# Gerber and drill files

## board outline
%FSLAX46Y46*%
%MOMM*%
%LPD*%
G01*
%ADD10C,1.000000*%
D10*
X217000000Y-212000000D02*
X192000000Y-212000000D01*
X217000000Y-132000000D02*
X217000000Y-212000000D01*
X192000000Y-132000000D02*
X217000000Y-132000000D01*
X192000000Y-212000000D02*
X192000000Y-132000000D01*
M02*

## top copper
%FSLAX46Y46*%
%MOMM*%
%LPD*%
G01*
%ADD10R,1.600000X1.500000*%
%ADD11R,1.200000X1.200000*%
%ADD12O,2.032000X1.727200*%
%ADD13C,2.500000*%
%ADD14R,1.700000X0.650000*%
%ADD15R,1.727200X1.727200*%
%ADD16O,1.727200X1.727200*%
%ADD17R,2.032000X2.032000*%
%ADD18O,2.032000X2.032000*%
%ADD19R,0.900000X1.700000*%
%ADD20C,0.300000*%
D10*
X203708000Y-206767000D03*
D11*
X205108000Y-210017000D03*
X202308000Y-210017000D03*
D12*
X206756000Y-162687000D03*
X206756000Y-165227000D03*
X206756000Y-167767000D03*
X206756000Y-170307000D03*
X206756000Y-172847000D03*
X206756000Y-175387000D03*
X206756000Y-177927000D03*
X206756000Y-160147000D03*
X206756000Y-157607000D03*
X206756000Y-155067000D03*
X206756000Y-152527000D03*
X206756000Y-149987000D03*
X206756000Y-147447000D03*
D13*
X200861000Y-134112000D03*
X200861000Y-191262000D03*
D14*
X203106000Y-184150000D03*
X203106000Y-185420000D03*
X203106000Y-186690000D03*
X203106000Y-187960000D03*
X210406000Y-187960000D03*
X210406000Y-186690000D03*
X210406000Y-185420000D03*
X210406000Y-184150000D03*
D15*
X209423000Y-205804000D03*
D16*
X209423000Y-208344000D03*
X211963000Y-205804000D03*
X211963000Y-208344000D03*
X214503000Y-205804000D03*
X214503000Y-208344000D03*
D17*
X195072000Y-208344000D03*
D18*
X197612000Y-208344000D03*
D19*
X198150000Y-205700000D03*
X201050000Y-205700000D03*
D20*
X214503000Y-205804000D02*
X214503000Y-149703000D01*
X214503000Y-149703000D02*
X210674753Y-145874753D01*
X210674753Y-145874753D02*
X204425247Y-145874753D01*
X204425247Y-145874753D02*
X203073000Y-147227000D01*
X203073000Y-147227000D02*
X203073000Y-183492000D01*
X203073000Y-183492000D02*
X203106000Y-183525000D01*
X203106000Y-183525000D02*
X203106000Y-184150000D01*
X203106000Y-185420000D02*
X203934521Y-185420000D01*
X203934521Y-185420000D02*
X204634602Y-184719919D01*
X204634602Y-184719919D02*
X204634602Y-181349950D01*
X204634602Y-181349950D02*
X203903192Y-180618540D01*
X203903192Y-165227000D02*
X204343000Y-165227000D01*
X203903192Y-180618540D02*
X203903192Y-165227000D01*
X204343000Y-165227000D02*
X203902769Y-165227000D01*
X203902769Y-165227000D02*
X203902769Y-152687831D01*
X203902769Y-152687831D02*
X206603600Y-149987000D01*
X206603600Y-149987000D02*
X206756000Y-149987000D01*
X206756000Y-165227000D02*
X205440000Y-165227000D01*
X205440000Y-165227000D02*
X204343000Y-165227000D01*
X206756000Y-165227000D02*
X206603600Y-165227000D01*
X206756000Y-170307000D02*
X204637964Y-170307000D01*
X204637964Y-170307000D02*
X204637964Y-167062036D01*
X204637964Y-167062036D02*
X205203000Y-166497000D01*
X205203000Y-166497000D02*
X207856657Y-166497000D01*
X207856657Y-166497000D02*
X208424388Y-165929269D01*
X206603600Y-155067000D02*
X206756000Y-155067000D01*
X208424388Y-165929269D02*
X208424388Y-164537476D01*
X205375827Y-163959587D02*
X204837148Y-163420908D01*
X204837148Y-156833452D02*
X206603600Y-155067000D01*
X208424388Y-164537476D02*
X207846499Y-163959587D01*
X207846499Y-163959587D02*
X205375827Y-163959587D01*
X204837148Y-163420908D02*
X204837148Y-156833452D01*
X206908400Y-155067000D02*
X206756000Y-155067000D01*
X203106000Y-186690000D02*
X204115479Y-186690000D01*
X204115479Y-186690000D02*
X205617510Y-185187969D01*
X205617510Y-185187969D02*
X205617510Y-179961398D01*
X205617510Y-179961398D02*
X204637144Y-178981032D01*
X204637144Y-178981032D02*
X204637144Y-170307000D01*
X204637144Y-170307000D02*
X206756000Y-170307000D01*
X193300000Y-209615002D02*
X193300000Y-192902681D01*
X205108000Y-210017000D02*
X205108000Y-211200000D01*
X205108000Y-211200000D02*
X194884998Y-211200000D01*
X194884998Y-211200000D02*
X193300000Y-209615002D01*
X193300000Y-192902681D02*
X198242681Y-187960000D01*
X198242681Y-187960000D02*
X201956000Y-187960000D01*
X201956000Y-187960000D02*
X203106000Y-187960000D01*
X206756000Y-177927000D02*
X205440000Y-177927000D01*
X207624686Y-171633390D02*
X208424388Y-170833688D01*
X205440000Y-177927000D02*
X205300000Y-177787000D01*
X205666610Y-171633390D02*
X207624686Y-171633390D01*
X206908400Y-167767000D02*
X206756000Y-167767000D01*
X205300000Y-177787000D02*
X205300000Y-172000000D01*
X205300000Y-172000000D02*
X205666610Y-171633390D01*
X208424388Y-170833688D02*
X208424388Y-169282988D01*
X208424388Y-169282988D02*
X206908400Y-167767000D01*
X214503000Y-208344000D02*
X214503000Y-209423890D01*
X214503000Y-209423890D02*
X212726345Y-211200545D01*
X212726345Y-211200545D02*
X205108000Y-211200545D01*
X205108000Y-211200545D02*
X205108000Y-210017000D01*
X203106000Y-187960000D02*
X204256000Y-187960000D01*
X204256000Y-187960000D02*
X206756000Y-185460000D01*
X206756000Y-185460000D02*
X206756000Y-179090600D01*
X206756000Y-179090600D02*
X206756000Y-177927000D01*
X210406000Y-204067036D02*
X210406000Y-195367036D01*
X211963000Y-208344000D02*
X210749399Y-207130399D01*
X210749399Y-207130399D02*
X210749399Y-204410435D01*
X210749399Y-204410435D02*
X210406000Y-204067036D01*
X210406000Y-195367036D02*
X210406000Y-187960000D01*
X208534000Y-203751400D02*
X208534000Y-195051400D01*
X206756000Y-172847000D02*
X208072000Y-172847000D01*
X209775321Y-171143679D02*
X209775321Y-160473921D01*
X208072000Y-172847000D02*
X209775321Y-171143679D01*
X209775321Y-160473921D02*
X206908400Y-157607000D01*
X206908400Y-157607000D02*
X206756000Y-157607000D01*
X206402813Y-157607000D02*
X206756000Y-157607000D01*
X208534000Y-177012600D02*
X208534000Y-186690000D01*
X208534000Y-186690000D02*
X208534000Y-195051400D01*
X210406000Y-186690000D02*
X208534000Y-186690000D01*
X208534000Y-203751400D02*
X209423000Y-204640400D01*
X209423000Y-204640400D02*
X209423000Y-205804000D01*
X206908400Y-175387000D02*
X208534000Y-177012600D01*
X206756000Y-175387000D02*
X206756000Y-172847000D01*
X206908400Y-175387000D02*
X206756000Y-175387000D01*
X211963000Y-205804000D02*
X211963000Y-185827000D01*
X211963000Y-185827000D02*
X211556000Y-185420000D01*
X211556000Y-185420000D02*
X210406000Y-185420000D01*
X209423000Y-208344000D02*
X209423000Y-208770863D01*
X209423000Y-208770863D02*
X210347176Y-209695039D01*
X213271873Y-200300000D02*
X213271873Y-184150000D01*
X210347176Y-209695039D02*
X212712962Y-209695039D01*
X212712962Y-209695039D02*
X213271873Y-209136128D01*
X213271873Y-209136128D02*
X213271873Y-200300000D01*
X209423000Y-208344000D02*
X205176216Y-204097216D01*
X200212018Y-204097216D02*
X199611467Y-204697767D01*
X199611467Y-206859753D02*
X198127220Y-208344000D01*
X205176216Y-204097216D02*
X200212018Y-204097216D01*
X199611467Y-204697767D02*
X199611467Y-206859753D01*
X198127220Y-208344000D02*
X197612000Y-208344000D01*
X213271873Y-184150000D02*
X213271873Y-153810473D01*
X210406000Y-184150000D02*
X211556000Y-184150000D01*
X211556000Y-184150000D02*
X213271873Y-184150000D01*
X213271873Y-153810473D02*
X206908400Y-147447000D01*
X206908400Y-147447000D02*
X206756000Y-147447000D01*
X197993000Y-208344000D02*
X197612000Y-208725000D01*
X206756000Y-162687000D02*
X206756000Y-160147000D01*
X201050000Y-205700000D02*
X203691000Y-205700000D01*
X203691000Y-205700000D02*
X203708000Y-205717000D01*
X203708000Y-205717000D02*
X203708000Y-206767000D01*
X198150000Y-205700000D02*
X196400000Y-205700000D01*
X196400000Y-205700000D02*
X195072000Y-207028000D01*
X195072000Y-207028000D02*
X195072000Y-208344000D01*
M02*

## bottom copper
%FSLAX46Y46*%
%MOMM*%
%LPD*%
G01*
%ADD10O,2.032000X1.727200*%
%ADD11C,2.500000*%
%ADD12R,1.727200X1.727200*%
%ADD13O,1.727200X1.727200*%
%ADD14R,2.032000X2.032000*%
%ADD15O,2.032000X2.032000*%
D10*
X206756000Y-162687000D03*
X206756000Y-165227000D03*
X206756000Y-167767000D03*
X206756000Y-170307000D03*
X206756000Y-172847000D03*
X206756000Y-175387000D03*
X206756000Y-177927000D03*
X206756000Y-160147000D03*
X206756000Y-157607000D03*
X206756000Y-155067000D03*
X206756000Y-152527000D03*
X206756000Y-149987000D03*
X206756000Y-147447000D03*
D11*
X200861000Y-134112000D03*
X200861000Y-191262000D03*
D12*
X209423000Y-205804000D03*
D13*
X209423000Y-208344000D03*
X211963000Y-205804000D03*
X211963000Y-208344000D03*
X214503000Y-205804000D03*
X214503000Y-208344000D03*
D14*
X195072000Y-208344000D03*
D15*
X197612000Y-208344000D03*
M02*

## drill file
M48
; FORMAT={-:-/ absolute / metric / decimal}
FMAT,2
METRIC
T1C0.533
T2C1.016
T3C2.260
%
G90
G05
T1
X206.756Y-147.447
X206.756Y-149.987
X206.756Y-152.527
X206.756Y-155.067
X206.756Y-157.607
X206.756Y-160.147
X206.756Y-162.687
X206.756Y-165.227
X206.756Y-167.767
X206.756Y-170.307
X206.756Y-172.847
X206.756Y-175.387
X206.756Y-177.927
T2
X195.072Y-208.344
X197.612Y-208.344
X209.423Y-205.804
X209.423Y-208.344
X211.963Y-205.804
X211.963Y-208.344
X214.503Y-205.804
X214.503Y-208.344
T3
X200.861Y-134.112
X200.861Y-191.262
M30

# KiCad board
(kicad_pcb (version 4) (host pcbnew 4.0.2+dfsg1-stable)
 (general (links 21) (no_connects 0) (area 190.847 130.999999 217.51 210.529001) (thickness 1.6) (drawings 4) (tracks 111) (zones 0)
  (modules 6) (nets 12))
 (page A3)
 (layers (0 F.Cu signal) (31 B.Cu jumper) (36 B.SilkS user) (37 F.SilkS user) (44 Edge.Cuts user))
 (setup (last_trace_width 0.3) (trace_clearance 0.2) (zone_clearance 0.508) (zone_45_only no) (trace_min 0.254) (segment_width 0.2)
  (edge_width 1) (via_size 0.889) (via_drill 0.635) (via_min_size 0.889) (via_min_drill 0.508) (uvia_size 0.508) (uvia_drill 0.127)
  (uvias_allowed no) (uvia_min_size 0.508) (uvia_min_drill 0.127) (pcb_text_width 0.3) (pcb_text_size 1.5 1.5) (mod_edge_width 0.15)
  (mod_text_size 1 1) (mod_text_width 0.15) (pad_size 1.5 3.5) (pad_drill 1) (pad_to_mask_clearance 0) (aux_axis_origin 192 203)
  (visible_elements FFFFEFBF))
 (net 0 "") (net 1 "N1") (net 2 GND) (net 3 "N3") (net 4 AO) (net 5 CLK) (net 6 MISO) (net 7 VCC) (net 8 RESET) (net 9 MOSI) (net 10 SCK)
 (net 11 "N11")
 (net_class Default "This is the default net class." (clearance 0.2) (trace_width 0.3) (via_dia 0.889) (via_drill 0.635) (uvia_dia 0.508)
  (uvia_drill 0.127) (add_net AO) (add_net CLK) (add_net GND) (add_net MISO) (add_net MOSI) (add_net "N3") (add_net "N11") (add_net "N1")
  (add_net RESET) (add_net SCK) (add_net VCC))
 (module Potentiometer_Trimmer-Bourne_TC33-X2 (layer F.Cu) (at 203.708 208.217)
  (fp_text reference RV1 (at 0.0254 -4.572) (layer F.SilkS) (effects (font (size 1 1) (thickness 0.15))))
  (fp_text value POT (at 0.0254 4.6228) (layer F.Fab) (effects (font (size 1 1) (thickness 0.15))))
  (pad 2 smd rect (at 0 -1.45) (size 1.6 1.5) (layers F.Cu) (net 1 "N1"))
  (pad 3 smd rect (at 1.4 1.8) (size 1.2 1.2) (layers F.Cu) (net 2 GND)) (pad 1 smd rect (at -1.4 1.8) (size 1.2 1.2) (layers F.Cu)))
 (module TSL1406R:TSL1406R (layer B.Cu) (at 200.861 162.687)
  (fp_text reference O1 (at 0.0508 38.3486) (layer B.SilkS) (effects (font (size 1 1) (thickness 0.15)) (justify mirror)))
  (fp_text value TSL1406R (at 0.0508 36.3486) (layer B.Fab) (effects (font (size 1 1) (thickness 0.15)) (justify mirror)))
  (pad 7 thru_hole oval (at 5.895 0) (size 2.032 1.7272) (drill 0.533) (layers *.Cu *.Mask B.SilkS) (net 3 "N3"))
  (pad 6 thru_hole oval (at 5.895 2.54) (size 2.032 1.7272) (drill 0.533) (layers *.Cu *.Mask B.SilkS) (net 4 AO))
  (pad 5 thru_hole oval (at 5.895 5.08) (size 2.032 1.7272) (drill 0.533) (layers *.Cu *.Mask B.SilkS) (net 2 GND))
  (pad 4 thru_hole oval (at 5.895 7.62) (size 2.032 1.7272) (drill 0.533) (layers *.Cu *.Mask B.SilkS) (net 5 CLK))
  (pad 3 thru_hole oval (at 5.895 10.16) (size 2.032 1.7272) (drill 0.533) (layers *.Cu *.Mask B.SilkS) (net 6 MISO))
  (pad 2 thru_hole oval (at 5.895 12.7) (size 2.032 1.7272) (drill 0.533) (layers *.Cu *.Mask B.SilkS) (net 6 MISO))
  (pad 1 thru_hole oval (at 5.895 15.24) (size 2.032 1.7272) (drill 0.533) (layers *.Cu *.Mask B.SilkS) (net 2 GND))
  (pad 8 thru_hole oval (at 5.895 -2.54) (size 2.032 1.7272) (drill 0.533) (layers *.Cu *.Mask B.SilkS) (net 3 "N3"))
  (pad 9 thru_hole oval (at 5.895 -5.08) (size 2.032 1.7272) (drill 0.533) (layers *.Cu *.Mask B.SilkS) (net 6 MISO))
  (pad 10 thru_hole oval (at 5.895 -7.62) (size 2.032 1.7272) (drill 0.533) (layers *.Cu *.Mask B.SilkS) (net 5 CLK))
  (pad 11 thru_hole oval (at 5.895 -10.16) (size 2.032 1.7272) (drill 0.533) (layers *.Cu *.Mask B.SilkS))
  (pad 12 thru_hole oval (at 5.895 -12.7) (size 2.032 1.7272) (drill 0.533) (layers *.Cu *.Mask B.SilkS) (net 4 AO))
  (pad 13 thru_hole oval (at 5.895 -15.24) (size 2.032 1.7272) (drill 0.533) (layers *.Cu *.Mask B.SilkS) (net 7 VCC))
  (pad 0 thru_hole circle (at 0 -28.575) (size 2.5 2.5) (drill 2.26) (layers *.Cu *.Mask B.SilkS))
  (pad 0 thru_hole circle (at 0 28.575) (size 2.5 2.5) (drill 2.26) (layers *.Cu *.Mask B.SilkS)))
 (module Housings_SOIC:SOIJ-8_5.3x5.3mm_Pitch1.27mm (layer F.Cu) (at 206.756 186.055)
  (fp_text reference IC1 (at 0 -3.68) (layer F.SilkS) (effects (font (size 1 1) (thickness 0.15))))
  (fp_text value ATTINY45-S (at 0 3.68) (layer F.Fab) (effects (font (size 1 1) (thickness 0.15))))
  (pad 1 smd rect (at -3.65 -1.905) (size 1.7 0.65) (layers F.Cu) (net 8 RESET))
  (pad 2 smd rect (at -3.65 -0.635) (size 1.7 0.65) (layers F.Cu) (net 4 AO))
  (pad 3 smd rect (at -3.65 0.635) (size 1.7 0.65) (layers F.Cu) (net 5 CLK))
  (pad 4 smd rect (at -3.65 1.905) (size 1.7 0.65) (layers F.Cu) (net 2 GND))
  (pad 5 smd rect (at 3.65 1.905) (size 1.7 0.65) (layers F.Cu) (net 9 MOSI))
  (pad 6 smd rect (at 3.65 0.635) (size 1.7 0.65) (layers F.Cu) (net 6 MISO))
  (pad 7 smd rect (at 3.65 -0.635) (size 1.7 0.65) (layers F.Cu) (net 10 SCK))
  (pad 8 smd rect (at 3.65 -1.905) (size 1.7 0.65) (layers F.Cu) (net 7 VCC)))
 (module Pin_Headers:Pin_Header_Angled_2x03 (layer B.Cu) (at 209.423 205.804 270)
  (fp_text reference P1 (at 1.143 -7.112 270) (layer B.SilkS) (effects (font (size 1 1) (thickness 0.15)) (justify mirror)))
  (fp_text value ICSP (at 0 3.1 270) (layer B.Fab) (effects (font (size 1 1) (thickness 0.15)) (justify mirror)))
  (pad 1 thru_hole rect (at 0 0 270) (size 1.7272 1.7272) (drill 1.016) (layers *.Cu *.Mask B.SilkS) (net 6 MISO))
  (pad 2 thru_hole oval (at 2.54 0 270) (size 1.7272 1.7272) (drill 1.016) (layers *.Cu *.Mask B.SilkS) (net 7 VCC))
  (pad 3 thru_hole oval (at 0 -2.54 270) (size 1.7272 1.7272) (drill 1.016) (layers *.Cu *.Mask B.SilkS) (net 10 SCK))
  (pad 4 thru_hole oval (at 2.54 -2.54 270) (size 1.7272 1.7272) (drill 1.016) (layers *.Cu *.Mask B.SilkS) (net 9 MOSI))
  (pad 5 thru_hole oval (at 0 -5.08 270) (size 1.7272 1.7272) (drill 1.016) (layers *.Cu *.Mask B.SilkS) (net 8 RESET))
  (pad 6 thru_hole oval (at 2.54 -5.08 270) (size 1.7272 1.7272) (drill 1.016) (layers *.Cu *.Mask B.SilkS) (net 2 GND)))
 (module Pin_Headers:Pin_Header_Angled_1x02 (layer B.Cu) (at 195.072 208.344 270)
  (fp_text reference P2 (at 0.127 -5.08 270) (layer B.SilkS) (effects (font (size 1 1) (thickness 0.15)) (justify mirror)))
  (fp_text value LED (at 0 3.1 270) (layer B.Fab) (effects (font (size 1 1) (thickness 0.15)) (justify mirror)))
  (pad 1 thru_hole rect (at 0 0 270) (size 2.032 2.032) (drill 1.016) (layers *.Cu *.Mask B.SilkS) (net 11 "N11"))
  (pad 2 thru_hole oval (at 0 -2.54 270) (size 2.032 2.032) (drill 1.016) (layers *.Cu *.Mask B.SilkS) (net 7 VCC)))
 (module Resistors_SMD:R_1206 (layer F.Cu) (at 199.6 205.7)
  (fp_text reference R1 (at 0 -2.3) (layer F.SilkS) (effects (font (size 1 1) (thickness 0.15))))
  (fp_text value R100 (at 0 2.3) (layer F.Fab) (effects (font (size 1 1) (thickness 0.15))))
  (pad 1 smd rect (at -1.45 0) (size 0.9 1.7) (layers F.Cu) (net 11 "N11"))
  (pad 2 smd rect (at 1.45 0) (size 0.9 1.7) (layers F.Cu) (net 1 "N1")))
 (gr_line (start 217 212) (end 192 212) (layer Edge.Cuts) (width 1))
 (gr_line (start 217 132) (end 217 212) (layer Edge.Cuts) (width 1))
 (gr_line (start 192 132) (end 217 132) (layer Edge.Cuts) (width 1))
 (gr_line (start 192 212) (end 192 132) (layer Edge.Cuts) (width 1))
 (segment (start 214.503 205.804) (end 214.503 149.703) (width 0.3) (layer F.Cu) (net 8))
 (segment (start 214.503 149.703) (end 210.674753 145.874753) (width 0.3) (layer F.Cu) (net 8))
 (segment (start 210.674753 145.874753) (end 204.425247 145.874753) (width 0.3) (layer F.Cu) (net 8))
 (segment (start 204.425247 145.874753) (end 203.073 147.227) (width 0.3) (layer F.Cu) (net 8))
 (segment (start 203.073 147.227) (end 203.073 183.492) (width 0.3) (layer F.Cu) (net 8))
 (segment (start 203.073 183.492) (end 203.106 183.525) (width 0.3) (layer F.Cu) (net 8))
 (segment (start 203.106 183.525) (end 203.106 184.15) (width 0.3) (layer F.Cu) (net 8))
 (segment (start 203.106 185.42) (end 203.934521 185.42) (width 0.3) (layer F.Cu) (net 4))
 (segment (start 203.934521 185.42) (end 204.634602 184.719919) (width 0.3) (layer F.Cu) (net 4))
 (segment (start 204.634602 184.719919) (end 204.634602 181.34995) (width 0.3) (layer F.Cu) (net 4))
 (segment (start 204.634602 181.34995) (end 203.903192 180.61854) (width 0.3) (layer F.Cu) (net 4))
 (segment (start 203.903192 165.227) (end 204.343 165.227) (width 0.3) (layer F.Cu) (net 4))
 (segment (start 203.903192 180.61854) (end 203.903192 165.227) (width 0.3) (layer F.Cu) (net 4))
 (segment (start 204.343 165.227) (end 203.902769 165.227) (width 0.3) (layer F.Cu) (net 4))
 (segment (start 203.902769 165.227) (end 203.902769 152.687831) (width 0.3) (layer F.Cu) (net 4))
 (segment (start 203.902769 152.687831) (end 206.6036 149.987) (width 0.3) (layer F.Cu) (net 4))
 (segment (start 206.6036 149.987) (end 206.756 149.987) (width 0.3) (layer F.Cu) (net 4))
 (segment (start 206.756 165.227) (end 205.44 165.227) (width 0.3) (layer F.Cu) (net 4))
 (segment (start 205.44 165.227) (end 204.343 165.227) (width 0.3) (layer F.Cu) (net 4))
 (segment (start 206.756 165.227) (end 206.6036 165.227) (width 0.3) (layer F.Cu) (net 4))
 (segment (start 206.756 170.307) (end 204.637964 170.307) (width 0.3) (layer F.Cu) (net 5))
 (segment (start 204.637964 170.307) (end 204.637964 167.062036) (width 0.3) (layer F.Cu) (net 5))
 (segment (start 204.637964 167.062036) (end 205.203 166.497) (width 0.3) (layer F.Cu) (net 5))
 (segment (start 205.203 166.497) (end 207.856657 166.497) (width 0.3) (layer F.Cu) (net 5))
 (segment (start 207.856657 166.497) (end 208.424388 165.929269) (width 0.3) (layer F.Cu) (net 5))
 (segment (start 206.6036 155.067) (end 206.756 155.067) (width 0.3) (layer F.Cu) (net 5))
 (segment (start 208.424388 165.929269) (end 208.424388 164.537476) (width 0.3) (layer F.Cu) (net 5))
 (segment (start 205.375827 163.959587) (end 204.837148 163.420908) (width 0.3) (layer F.Cu) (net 5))
 (segment (start 204.837148 156.833452) (end 206.6036 155.067) (width 0.3) (layer F.Cu) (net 5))
 (segment (start 208.424388 164.537476) (end 207.846499 163.959587) (width 0.3) (layer F.Cu) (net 5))
 (segment (start 207.846499 163.959587) (end 205.375827 163.959587) (width 0.3) (layer F.Cu) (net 5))
 (segment (start 204.837148 163.420908) (end 204.837148 156.833452) (width 0.3) (layer F.Cu) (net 5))
 (segment (start 206.9084 155.067) (end 206.756 155.067) (width 0.3) (layer F.Cu) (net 5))
 (segment (start 203.106 186.69) (end 204.115479 186.69) (width 0.3) (layer F.Cu) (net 5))
 (segment (start 204.115479 186.69) (end 205.61751 185.187969) (width 0.3) (layer F.Cu) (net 5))
 (segment (start 205.61751 185.187969) (end 205.61751 179.961398) (width 0.3) (layer F.Cu) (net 5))
 (segment (start 205.61751 179.961398) (end 204.637144 178.981032) (width 0.3) (layer F.Cu) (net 5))
 (segment (start 204.637144 178.981032) (end 204.637144 170.307) (width 0.3) (layer F.Cu) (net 5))
 (segment (start 204.637144 170.307) (end 206.756 170.307) (width 0.3) (layer F.Cu) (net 5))
 (segment (start 193.3 209.615002) (end 193.3 192.902681) (width 0.3) (layer F.Cu) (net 2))
 (segment (start 205.108 210.017) (end 205.108 211.2) (width 0.3) (layer F.Cu) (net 2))
 (segment (start 205.108 211.2) (end 194.884998 211.2) (width 0.3) (layer F.Cu) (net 2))
 (segment (start 194.884998 211.2) (end 193.3 209.615002) (width 0.3) (layer F.Cu) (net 2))
 (segment (start 193.3 192.902681) (end 198.242681 187.96) (width 0.3) (layer F.Cu) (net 2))
 (segment (start 198.242681 187.96) (end 201.956 187.96) (width 0.3) (layer F.Cu) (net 2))
 (segment (start 201.956 187.96) (end 203.106 187.96) (width 0.3) (layer F.Cu) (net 2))
 (segment (start 206.756 177.927) (end 205.44 177.927) (width 0.3) (layer F.Cu) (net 2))
 (segment (start 207.624686 171.63339) (end 208.424388 170.833688) (width 0.3) (layer F.Cu) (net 2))
 (segment (start 205.44 177.927) (end 205.3 177.787) (width 0.3) (layer F.Cu) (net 2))
 (segment (start 205.66661 171.63339) (end 207.624686 171.63339) (width 0.3) (layer F.Cu) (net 2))
 (segment (start 206.9084 167.767) (end 206.756 167.767) (width 0.3) (layer F.Cu) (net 2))
 (segment (start 205.3 177.787) (end 205.3 172) (width 0.3) (layer F.Cu) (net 2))
 (segment (start 205.3 172) (end 205.66661 171.63339) (width 0.3) (layer F.Cu) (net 2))
 (segment (start 208.424388 170.833688) (end 208.424388 169.282988) (width 0.3) (layer F.Cu) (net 2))
 (segment (start 208.424388 169.282988) (end 206.9084 167.767) (width 0.3) (layer F.Cu) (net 2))
 (segment (start 214.503 208.344) (end 214.503 209.42389) (width 0.3) (layer F.Cu) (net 2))
 (segment (start 214.503 209.42389) (end 212.726345 211.200545) (width 0.3) (layer F.Cu) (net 2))
 (segment (start 212.726345 211.200545) (end 205.108 211.200545) (width 0.3) (layer F.Cu) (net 2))
 (segment (start 205.108 211.200545) (end 205.108 210.017) (width 0.3) (layer F.Cu) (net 2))
 (segment (start 203.106 187.96) (end 204.256 187.96) (width 0.3) (layer F.Cu) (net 2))
 (segment (start 204.256 187.96) (end 206.756 185.46) (width 0.3) (layer F.Cu) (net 2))
 (segment (start 206.756 185.46) (end 206.756 179.0906) (width 0.3) (layer F.Cu) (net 2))
 (segment (start 206.756 179.0906) (end 206.756 177.927) (width 0.3) (layer F.Cu) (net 2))
 (segment (start 210.406 204.067036) (end 210.406 195.367036) (width 0.3) (layer F.Cu) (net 9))
 (segment (start 211.963 208.344) (end 210.749399 207.130399) (width 0.3) (layer F.Cu) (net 9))
 (segment (start 210.749399 207.130399) (end 210.749399 204.410435) (width 0.3) (layer F.Cu) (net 9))
 (segment (start 210.749399 204.410435) (end 210.406 204.067036) (width 0.3) (layer F.Cu) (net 9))
 (segment (start 210.406 195.367036) (end 210.406 187.96) (width 0.3) (layer F.Cu) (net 9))
 (segment (start 208.534 203.7514) (end 208.534 195.0514) (width 0.3) (layer F.Cu) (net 6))
 (segment (start 206.756 172.847) (end 208.072 172.847) (width 0.3) (layer F.Cu) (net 6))
 (segment (start 209.775321 171.143679) (end 209.775321 160.473921) (width 0.3) (layer F.Cu) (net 6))
 (segment (start 208.072 172.847) (end 209.775321 171.143679) (width 0.3) (layer F.Cu) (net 6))
 (segment (start 209.775321 160.473921) (end 206.9084 157.607) (width 0.3) (layer F.Cu) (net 6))
 (segment (start 206.9084 157.607) (end 206.756 157.607) (width 0.3) (layer F.Cu) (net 6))
 (segment (start 206.402813 157.607) (end 206.756 157.607) (width 0.3) (layer F.Cu) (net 6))
 (segment (start 208.534 177.0126) (end 208.534 186.69) (width 0.3) (layer F.Cu) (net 6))
 (segment (start 208.534 186.69) (end 208.534 195.0514) (width 0.3) (layer F.Cu) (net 6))
 (segment (start 210.406 186.69) (end 208.534 186.69) (width 0.3) (layer F.Cu) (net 6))
 (segment (start 208.534 203.7514) (end 209.423 204.6404) (width 0.3) (layer F.Cu) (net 6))
 (segment (start 209.423 204.6404) (end 209.423 205.804) (width 0.3) (layer F.Cu) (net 6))
 (segment (start 206.9084 175.387) (end 208.534 177.0126) (width 0.3) (layer F.Cu) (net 6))
 (segment (start 206.756 175.387) (end 206.756 172.847) (width 0.3) (layer F.Cu) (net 6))
 (segment (start 206.9084 175.387) (end 206.756 175.387) (width 0.3) (layer F.Cu) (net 6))
 (segment (start 211.963 205.804) (end 211.963 185.827) (width 0.3) (layer F.Cu) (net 10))
 (segment (start 211.963 185.827) (end 211.556 185.42) (width 0.3) (layer F.Cu) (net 10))
 (segment (start 211.556 185.42) (end 210.406 185.42) (width 0.3) (layer F.Cu) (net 10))
 (segment (start 209.423 208.344) (end 209.423 208.770863) (width 0.3) (layer F.Cu) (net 7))
 (segment (start 209.423 208.770863) (end 210.347176 209.695039) (width 0.3) (layer F.Cu) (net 7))
 (segment (start 213.271873 200.3) (end 213.271873 184.15) (width 0.3) (layer F.Cu) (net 7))
 (segment (start 210.347176 209.695039) (end 212.712962 209.695039) (width 0.3) (layer F.Cu) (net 7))
 (segment (start 212.712962 209.695039) (end 213.271873 209.136128) (width 0.3) (layer F.Cu) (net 7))
 (segment (start 213.271873 209.136128) (end 213.271873 200.3) (width 0.3) (layer F.Cu) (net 7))
 (segment (start 209.423 208.344) (end 205.176216 204.097216) (width 0.3) (layer F.Cu) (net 7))
 (segment (start 200.212018 204.097216) (end 199.611467 204.697767) (width 0.3) (layer F.Cu) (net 7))
 (segment (start 199.611467 206.859753) (end 198.12722 208.344) (width 0.3) (layer F.Cu) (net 7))
 (segment (start 205.176216 204.097216) (end 200.212018 204.097216) (width 0.3) (layer F.Cu) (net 7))
 (segment (start 199.611467 204.697767) (end 199.611467 206.859753) (width 0.3) (layer F.Cu) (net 7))
 (segment (start 198.12722 208.344) (end 197.612 208.344) (width 0.3) (layer F.Cu) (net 7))
 (segment (start 213.271873 184.15) (end 213.271873 153.810473) (width 0.3) (layer F.Cu) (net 7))
 (segment (start 210.406 184.15) (end 211.556 184.15) (width 0.3) (layer F.Cu) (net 7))
 (segment (start 211.556 184.15) (end 213.271873 184.15) (width 0.3) (layer F.Cu) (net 7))
 (segment (start 213.271873 153.810473) (end 206.9084 147.447) (width 0.3) (layer F.Cu) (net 7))
 (segment (start 206.9084 147.447) (end 206.756 147.447) (width 0.3) (layer F.Cu) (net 7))
 (segment (start 197.993 208.344) (end 197.612 208.725) (width 0.3) (layer F.Cu) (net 7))
 (segment (start 206.756 162.687) (end 206.756 160.147) (width 0.3) (layer F.Cu) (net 3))
 (segment (start 201.05 205.7) (end 203.691 205.7) (width 0.3) (layer F.Cu) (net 1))
 (segment (start 203.691 205.7) (end 203.708 205.717) (width 0.3) (layer F.Cu) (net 1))
 (segment (start 203.708 205.717) (end 203.708 206.767) (width 0.3) (layer F.Cu) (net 1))
 (segment (start 198.15 205.7) (end 196.4 205.7) (width 0.3) (layer F.Cu) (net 11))
 (segment (start 196.4 205.7) (end 195.072 207.028) (width 0.3) (layer F.Cu) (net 11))
 (segment (start 195.072 207.028) (end 195.072 208.344) (width 0.3) (layer F.Cu) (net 11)))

